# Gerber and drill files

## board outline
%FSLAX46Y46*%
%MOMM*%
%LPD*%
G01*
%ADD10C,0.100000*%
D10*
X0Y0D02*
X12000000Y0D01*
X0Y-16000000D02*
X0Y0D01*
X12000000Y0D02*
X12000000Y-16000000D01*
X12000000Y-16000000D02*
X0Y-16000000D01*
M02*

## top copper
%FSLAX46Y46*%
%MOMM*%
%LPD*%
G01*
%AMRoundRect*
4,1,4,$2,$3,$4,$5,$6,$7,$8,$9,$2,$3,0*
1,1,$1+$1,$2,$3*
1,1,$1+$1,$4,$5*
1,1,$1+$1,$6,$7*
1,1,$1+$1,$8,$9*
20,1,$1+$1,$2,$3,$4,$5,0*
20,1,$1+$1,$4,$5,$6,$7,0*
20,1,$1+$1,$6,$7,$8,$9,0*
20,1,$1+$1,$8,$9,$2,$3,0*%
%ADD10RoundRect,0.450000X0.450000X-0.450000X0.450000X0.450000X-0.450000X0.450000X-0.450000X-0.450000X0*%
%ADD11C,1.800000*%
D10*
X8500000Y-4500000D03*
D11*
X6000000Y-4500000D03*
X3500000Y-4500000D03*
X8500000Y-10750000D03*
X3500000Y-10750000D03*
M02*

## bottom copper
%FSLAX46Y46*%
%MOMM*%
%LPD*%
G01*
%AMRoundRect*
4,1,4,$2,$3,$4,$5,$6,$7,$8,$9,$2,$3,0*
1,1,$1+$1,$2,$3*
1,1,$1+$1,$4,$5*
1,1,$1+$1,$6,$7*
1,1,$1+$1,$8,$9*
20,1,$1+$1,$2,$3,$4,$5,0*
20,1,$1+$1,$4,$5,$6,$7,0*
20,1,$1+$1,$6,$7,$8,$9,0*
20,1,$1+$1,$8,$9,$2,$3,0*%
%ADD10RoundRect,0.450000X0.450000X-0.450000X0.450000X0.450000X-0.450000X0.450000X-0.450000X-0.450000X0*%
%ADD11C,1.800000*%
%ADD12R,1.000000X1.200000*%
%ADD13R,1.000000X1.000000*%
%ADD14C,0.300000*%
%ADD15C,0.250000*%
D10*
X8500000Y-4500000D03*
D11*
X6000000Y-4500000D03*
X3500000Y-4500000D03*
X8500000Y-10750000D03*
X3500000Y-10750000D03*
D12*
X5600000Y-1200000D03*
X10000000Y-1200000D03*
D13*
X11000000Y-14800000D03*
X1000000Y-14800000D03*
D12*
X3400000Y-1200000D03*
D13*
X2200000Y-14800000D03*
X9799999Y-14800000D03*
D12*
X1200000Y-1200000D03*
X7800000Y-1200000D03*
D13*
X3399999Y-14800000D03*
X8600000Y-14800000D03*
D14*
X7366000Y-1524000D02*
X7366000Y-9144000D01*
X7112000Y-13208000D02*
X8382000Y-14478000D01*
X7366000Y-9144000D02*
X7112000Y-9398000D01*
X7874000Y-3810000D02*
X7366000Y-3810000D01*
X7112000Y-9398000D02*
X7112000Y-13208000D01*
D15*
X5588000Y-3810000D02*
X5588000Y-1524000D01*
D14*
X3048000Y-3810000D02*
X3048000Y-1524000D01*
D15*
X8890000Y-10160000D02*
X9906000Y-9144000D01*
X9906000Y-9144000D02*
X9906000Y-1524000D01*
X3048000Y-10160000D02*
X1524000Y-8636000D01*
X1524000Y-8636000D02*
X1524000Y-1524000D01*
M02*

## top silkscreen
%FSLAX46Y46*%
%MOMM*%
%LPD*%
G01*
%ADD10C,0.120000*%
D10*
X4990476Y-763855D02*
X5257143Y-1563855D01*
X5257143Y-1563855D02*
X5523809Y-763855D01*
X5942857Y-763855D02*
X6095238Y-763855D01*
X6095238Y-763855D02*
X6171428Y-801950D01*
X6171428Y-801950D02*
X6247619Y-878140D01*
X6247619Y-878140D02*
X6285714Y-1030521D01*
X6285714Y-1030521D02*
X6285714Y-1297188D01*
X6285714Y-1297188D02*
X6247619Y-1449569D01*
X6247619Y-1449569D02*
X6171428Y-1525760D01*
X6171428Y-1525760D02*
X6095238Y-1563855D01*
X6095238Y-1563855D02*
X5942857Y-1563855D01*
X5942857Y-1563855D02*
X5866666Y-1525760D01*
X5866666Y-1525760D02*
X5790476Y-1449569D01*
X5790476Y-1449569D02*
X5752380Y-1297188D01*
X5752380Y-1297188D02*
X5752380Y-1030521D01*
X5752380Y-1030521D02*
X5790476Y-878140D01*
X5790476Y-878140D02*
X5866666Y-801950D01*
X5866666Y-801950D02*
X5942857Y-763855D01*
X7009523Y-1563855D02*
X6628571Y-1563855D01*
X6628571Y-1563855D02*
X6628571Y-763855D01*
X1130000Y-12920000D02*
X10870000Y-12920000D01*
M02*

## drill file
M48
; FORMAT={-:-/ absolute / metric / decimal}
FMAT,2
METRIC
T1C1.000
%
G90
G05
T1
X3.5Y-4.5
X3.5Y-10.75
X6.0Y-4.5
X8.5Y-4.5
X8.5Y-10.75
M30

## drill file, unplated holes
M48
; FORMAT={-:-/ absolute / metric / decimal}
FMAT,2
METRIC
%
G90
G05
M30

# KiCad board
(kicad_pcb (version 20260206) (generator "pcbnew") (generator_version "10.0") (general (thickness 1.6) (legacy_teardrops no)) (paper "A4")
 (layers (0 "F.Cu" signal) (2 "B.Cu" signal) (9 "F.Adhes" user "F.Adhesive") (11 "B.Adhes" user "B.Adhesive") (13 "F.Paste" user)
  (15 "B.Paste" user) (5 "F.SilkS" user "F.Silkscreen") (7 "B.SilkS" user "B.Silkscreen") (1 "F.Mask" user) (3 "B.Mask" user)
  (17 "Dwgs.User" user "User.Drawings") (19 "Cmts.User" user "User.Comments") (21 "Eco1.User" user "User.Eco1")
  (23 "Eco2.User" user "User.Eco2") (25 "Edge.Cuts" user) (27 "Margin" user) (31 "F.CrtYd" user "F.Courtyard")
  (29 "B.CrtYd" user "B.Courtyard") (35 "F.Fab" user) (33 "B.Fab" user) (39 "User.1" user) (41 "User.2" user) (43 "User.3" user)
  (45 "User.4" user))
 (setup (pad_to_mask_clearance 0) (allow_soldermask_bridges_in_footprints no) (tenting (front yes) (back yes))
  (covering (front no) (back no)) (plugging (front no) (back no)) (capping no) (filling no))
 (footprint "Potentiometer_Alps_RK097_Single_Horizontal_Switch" (layer "F.Cu") (at 8.5 4.5 -90)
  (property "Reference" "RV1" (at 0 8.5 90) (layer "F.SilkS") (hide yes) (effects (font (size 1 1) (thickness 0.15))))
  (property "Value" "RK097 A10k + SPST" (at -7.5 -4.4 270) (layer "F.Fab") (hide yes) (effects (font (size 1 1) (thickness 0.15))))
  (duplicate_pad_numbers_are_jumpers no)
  (fp_line (start 8.42 7.37) (end 8.42 -2.37) (stroke (width 0.12) (type solid)) (layer "F.SilkS"))
  (pad "1" thru_hole roundrect (at 0 0 90) (size 1.8 1.8) (drill 1) (layers "*.Cu" "*.Mask") (remove_unused_layers no)
   (roundrect_rratio 0.25) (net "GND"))
  (pad "2" thru_hole circle (at 0 2.5 90) (size 1.8 1.8) (drill 1) (layers "*.Cu" "*.Mask") (remove_unused_layers no) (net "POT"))
  (pad "3" thru_hole circle (at 0 5 90) (size 1.8 1.8) (drill 1) (layers "*.Cu" "*.Mask") (remove_unused_layers no) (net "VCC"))
  (pad "4" thru_hole circle (at 6.25 0 90) (size 1.8 1.8) (drill 1) (layers "*.Cu" "*.Mask") (remove_unused_layers no) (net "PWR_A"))
  (pad "5" thru_hole circle (at 6.25 5 90) (size 1.8 1.8) (drill 1) (layers "*.Cu" "*.Mask") (remove_unused_layers no) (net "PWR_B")))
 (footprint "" (layer "B.Cu") (at 5.6 1.2 180)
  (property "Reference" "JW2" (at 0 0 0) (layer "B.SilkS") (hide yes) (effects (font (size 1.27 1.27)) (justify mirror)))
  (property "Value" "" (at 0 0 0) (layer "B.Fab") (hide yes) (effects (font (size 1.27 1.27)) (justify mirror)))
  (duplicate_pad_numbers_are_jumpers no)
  (pad "1" smd rect (at 0 0 180) (size 1 1.2) (layers "B.Cu" "B.Mask" "B.Paste") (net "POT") (thermal_bridge_angle 45)))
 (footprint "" (layer "B.Cu") (at 10 1.2 180)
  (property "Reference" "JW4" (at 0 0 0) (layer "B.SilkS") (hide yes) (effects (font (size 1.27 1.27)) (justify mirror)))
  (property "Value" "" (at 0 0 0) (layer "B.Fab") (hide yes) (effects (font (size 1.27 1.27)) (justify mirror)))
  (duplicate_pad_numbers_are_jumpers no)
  (pad "1" smd rect (at 0 0 180) (size 1 1.2) (layers "B.Cu" "B.Mask" "B.Paste") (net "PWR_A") (thermal_bridge_angle 45)))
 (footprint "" (layer "B.Cu") (at 11 14.8 180)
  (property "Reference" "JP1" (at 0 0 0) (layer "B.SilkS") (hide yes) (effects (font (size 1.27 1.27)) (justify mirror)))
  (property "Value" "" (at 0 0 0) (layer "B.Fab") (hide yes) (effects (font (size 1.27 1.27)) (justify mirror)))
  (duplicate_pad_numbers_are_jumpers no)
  (pad "1" smd rect (at 0 0 180) (size 1 1) (layers "B.Cu" "B.Mask" "B.Paste") (thermal_bridge_angle 45)))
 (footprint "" (layer "B.Cu") (at 1 14.8 180)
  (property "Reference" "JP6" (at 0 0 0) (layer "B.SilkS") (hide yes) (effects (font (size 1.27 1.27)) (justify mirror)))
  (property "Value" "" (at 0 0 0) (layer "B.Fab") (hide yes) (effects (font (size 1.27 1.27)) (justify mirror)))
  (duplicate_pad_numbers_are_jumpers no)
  (pad "1" smd rect (at 0 0 180) (size 1 1) (layers "B.Cu" "B.Mask" "B.Paste") (thermal_bridge_angle 45)))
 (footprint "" (layer "B.Cu") (at 3.4 1.2 180)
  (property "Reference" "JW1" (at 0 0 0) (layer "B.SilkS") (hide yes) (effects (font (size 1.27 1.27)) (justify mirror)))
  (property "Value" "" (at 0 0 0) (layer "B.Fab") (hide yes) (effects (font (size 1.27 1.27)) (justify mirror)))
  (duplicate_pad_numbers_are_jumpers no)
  (pad "1" smd rect (at 0 0 180) (size 1 1.2) (layers "B.Cu" "B.Mask" "B.Paste") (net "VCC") (thermal_bridge_angle 45)))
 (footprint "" (layer "B.Cu") (at 2.2 14.8 180)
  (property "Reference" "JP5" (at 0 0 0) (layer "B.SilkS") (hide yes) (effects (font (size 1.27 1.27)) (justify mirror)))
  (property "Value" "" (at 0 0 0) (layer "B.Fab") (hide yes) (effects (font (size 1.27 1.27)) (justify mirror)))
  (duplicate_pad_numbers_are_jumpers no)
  (pad "1" smd rect (at 0 0 180) (size 1 1) (layers "B.Cu" "B.Mask" "B.Paste") (thermal_bridge_angle 45)))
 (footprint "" (layer "B.Cu") (at 9.799999 14.8 180)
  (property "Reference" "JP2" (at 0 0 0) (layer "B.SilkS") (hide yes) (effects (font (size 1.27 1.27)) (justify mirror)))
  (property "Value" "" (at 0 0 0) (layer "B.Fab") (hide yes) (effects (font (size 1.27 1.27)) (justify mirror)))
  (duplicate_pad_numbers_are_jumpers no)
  (pad "1" smd rect (at 0 0 180) (size 1 1) (layers "B.Cu" "B.Mask" "B.Paste") (thermal_bridge_angle 45)))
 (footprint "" (layer "B.Cu") (at 1.2 1.2 180)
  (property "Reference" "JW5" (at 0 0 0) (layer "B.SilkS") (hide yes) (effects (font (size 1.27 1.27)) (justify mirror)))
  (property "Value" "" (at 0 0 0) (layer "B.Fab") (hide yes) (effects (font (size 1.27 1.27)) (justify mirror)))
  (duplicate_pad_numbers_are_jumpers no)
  (pad "1" smd rect (at 0 0 180) (size 1 1.2) (layers "B.Cu" "B.Mask" "B.Paste") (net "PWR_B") (thermal_bridge_angle 45)))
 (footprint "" (layer "B.Cu") (at 7.8 1.2 180)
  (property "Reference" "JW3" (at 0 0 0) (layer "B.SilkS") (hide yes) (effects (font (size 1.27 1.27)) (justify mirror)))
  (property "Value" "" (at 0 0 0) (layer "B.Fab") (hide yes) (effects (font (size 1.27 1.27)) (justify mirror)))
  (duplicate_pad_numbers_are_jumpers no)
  (pad "1" smd rect (at 0 0 180) (size 1 1.2) (layers "B.Cu" "B.Mask" "B.Paste") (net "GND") (thermal_bridge_angle 45)))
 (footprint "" (layer "B.Cu") (at 3.399999 14.8 180)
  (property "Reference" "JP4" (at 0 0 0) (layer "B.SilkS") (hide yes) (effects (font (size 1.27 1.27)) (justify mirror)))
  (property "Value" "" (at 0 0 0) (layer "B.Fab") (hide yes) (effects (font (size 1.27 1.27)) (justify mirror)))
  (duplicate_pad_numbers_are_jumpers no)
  (pad "1" smd rect (at 0 0 180) (size 1 1) (layers "B.Cu" "B.Mask" "B.Paste") (thermal_bridge_angle 45)))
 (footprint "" (layer "B.Cu") (at 8.6 14.8 180)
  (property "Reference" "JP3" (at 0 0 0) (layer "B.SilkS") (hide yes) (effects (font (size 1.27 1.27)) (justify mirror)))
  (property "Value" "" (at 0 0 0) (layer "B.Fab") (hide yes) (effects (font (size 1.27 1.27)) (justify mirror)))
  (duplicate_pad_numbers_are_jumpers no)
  (pad "1" smd rect (at 0 0 180) (size 1 1) (layers "B.Cu" "B.Mask" "B.Paste") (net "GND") (thermal_bridge_angle 45)))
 (gr_line (start 0 0) (end 12 0) (stroke (width 0.1) (type default)) (layer "Edge.Cuts"))
 (gr_line (start 0 16) (end 0 0) (stroke (width 0.1) (type default)) (layer "Edge.Cuts"))
 (gr_line (start 12 0) (end 12 16) (stroke (width 0.1) (type default)) (layer "Edge.Cuts"))
 (gr_line (start 12 16) (end 0 16) (stroke (width 0.1) (type default)) (layer "Edge.Cuts"))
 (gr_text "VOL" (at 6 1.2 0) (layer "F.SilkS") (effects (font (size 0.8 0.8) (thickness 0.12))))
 (segment (start 7.366 1.524) (end 7.366 9.144) (width 0.3) (layer "B.Cu") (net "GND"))
 (segment (start 7.112 13.208) (end 8.382 14.478) (width 0.3) (layer "B.Cu") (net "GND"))
 (segment (start 7.366 9.144) (end 7.112 9.398) (width 0.3) (layer "B.Cu") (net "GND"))
 (segment (start 7.874 3.81) (end 7.366 3.81) (width 0.3) (layer "B.Cu") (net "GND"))
 (segment (start 7.112 9.398) (end 7.112 13.208) (width 0.3) (layer "B.Cu") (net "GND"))
 (segment (start 5.588 3.81) (end 5.588 1.524) (width 0.25) (layer "B.Cu") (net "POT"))
 (segment (start 3.048 3.81) (end 3.048 1.524) (width 0.3) (layer "B.Cu") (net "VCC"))
 (segment (start 8.89 10.16) (end 9.906 9.144) (width 0.25) (layer "B.Cu") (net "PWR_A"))
 (segment (start 9.906 9.144) (end 9.906 1.524) (width 0.25) (layer "B.Cu") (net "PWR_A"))
 (segment (start 3.048 10.16) (end 1.524 8.636) (width 0.25) (layer "B.Cu") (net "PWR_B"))
 (segment (start 1.524 8.636) (end 1.524 1.524) (width 0.25) (layer "B.Cu") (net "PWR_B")))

